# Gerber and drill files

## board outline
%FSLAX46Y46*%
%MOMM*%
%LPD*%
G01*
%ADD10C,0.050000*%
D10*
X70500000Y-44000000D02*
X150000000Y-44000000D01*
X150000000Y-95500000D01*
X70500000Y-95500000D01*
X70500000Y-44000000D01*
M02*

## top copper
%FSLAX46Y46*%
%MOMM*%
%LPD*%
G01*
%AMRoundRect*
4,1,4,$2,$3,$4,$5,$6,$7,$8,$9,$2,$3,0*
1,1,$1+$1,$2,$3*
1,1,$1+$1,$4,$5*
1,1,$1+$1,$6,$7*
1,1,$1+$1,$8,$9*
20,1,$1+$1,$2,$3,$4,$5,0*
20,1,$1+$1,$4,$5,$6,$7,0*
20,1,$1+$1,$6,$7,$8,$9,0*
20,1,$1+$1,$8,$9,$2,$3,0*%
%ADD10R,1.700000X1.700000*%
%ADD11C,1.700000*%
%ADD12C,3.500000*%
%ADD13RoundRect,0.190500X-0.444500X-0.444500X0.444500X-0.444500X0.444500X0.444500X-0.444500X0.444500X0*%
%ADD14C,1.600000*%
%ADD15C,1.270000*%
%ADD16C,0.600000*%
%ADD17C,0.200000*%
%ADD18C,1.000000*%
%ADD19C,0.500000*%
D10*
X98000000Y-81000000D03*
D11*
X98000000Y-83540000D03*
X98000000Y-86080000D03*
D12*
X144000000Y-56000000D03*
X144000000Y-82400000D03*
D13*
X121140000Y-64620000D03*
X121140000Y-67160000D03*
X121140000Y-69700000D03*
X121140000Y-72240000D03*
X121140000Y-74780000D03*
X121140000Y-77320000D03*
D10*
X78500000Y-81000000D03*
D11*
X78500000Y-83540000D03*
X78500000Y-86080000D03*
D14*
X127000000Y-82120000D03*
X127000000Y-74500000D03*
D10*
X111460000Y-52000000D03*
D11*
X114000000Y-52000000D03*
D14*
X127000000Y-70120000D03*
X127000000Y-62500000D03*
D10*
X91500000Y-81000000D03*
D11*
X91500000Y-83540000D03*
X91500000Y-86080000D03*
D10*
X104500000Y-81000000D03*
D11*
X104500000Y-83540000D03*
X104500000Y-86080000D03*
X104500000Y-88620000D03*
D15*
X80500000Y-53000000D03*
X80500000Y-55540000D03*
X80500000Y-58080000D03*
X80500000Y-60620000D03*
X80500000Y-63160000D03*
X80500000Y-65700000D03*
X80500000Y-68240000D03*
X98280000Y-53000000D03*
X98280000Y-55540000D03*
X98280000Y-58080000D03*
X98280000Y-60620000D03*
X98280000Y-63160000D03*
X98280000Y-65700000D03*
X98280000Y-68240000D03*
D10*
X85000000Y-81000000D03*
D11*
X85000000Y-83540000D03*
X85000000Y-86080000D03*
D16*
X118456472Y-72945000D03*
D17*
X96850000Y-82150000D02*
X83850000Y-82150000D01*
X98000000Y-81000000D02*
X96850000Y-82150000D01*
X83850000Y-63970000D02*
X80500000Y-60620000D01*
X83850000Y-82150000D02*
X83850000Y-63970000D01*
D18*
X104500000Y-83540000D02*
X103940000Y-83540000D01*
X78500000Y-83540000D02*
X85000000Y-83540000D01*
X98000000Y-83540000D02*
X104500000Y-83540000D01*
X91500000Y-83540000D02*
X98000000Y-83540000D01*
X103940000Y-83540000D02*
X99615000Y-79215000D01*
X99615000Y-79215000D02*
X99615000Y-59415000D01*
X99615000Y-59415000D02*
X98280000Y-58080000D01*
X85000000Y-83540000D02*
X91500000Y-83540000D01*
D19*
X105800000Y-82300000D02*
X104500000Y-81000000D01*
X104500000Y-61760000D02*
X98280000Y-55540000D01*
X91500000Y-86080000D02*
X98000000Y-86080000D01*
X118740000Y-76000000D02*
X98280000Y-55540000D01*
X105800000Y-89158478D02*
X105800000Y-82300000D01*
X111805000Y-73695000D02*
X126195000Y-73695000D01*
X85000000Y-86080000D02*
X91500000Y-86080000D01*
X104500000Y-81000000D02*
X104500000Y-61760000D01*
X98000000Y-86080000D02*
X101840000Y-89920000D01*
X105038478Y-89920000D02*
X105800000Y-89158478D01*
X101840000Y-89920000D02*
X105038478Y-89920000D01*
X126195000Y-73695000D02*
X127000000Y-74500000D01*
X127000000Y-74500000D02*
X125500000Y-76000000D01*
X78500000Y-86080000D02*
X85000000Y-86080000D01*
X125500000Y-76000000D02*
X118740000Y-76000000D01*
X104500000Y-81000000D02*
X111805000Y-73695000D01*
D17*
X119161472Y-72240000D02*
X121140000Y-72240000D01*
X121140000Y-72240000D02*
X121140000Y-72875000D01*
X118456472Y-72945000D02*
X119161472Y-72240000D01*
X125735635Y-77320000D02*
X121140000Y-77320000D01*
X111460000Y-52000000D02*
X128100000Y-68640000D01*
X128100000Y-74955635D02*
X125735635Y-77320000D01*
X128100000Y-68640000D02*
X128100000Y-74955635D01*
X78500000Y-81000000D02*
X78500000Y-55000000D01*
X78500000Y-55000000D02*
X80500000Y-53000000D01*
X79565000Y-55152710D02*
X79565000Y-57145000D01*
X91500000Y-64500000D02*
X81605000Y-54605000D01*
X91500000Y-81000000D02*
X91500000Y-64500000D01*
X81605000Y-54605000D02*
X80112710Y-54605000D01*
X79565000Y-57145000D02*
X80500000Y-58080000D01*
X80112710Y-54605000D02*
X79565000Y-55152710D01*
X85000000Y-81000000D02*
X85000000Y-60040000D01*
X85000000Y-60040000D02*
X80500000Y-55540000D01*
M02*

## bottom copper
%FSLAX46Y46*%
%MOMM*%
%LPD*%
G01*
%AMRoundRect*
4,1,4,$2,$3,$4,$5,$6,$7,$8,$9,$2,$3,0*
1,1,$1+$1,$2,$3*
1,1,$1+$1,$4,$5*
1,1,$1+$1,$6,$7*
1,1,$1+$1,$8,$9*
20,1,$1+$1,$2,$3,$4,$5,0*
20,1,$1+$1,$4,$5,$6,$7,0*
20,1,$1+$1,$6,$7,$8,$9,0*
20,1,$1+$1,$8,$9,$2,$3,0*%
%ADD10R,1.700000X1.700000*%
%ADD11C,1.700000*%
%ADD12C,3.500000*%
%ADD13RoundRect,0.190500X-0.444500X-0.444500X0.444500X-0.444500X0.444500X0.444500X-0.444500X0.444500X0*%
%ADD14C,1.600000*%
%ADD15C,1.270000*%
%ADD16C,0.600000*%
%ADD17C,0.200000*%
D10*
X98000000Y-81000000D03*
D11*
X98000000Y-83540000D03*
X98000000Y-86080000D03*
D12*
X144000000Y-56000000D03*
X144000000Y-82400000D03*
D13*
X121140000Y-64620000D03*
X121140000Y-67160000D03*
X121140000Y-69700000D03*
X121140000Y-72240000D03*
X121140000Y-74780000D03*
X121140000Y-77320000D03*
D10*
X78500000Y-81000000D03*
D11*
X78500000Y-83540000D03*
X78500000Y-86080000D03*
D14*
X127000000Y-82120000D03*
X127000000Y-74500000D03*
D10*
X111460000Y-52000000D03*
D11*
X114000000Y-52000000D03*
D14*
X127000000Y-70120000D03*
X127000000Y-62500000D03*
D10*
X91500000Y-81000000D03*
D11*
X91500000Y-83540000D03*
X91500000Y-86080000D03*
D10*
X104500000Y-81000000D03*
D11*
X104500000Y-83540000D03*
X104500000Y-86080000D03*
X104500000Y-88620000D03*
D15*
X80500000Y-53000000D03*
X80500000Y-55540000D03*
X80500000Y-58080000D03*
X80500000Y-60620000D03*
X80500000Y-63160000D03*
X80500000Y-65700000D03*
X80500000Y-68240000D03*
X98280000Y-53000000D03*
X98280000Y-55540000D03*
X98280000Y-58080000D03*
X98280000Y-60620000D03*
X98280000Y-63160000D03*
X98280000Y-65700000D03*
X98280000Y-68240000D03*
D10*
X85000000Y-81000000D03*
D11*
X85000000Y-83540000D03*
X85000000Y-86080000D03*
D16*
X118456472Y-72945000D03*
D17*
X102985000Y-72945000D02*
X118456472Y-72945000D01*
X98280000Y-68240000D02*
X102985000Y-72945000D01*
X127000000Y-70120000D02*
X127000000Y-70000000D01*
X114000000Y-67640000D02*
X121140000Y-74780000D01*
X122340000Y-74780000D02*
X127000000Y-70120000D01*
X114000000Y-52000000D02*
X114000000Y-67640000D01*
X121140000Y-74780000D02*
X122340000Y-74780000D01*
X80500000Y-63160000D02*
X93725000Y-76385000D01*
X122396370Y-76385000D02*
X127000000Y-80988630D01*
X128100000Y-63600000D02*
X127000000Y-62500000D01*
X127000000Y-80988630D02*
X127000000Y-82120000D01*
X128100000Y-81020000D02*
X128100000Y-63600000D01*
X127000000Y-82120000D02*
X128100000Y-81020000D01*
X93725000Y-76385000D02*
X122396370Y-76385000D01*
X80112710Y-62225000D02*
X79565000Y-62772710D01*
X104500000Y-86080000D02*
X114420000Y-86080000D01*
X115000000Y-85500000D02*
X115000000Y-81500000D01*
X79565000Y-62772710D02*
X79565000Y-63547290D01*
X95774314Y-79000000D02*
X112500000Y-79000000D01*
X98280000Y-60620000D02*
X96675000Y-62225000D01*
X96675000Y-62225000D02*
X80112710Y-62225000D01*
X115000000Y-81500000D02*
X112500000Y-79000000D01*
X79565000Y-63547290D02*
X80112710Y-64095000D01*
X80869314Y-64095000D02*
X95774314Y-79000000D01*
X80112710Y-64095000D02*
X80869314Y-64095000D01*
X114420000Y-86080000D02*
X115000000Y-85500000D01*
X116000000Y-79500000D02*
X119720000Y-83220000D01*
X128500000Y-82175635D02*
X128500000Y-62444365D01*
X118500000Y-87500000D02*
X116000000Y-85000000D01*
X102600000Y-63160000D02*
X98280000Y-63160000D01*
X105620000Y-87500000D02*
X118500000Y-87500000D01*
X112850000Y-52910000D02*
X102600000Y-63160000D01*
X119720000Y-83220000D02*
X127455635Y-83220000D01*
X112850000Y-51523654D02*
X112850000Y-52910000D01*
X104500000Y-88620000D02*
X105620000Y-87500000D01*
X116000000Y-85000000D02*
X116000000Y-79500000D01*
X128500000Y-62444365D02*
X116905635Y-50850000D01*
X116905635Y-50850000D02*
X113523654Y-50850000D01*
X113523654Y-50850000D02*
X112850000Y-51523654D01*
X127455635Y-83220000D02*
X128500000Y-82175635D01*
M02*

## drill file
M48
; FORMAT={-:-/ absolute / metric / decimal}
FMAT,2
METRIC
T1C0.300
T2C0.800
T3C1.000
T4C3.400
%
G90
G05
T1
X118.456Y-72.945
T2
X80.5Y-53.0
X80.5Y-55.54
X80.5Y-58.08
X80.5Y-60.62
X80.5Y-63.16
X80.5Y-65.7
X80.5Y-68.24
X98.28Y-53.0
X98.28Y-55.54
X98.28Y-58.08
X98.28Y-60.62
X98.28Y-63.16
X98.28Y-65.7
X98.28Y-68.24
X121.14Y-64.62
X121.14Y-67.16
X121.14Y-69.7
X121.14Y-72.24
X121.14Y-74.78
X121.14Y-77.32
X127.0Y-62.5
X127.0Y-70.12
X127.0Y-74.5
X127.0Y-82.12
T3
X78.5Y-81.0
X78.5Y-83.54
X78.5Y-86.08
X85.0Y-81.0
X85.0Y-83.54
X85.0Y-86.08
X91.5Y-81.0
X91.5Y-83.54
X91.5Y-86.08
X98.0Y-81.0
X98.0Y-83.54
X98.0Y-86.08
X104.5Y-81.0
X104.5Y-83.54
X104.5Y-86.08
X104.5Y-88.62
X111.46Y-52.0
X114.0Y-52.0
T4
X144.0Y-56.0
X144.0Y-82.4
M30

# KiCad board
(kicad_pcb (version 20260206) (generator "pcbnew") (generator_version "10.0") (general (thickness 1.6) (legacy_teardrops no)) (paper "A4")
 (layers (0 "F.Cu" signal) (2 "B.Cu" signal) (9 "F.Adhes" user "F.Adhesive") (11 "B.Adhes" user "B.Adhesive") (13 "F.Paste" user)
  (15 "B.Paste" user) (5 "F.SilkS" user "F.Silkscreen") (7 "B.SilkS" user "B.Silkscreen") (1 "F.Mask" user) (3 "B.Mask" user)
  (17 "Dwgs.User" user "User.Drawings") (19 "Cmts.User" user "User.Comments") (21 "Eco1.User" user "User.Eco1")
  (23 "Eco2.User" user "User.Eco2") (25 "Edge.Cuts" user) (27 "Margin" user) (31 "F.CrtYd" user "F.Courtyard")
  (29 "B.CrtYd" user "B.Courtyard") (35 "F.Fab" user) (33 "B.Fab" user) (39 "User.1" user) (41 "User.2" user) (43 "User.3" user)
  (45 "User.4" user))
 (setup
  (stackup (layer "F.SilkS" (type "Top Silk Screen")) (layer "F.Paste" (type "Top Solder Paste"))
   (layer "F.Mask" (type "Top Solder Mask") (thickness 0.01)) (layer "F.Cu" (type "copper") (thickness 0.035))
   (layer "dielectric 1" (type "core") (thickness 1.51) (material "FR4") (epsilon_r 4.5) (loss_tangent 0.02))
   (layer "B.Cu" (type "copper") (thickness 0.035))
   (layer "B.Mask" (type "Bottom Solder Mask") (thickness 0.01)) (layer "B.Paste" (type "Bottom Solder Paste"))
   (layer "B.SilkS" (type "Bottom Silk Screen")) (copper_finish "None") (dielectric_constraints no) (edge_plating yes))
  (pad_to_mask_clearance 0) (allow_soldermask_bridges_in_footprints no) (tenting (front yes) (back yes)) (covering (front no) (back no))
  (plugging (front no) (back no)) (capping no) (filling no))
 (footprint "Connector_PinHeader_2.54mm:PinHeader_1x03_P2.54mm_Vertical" (layer "F.Cu") (at 98 81)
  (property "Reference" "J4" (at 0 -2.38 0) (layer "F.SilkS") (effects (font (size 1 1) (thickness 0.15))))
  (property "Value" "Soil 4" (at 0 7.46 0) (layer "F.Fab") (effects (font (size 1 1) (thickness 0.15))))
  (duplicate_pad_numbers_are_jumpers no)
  (pad "1" thru_hole rect (at 0 0) (size 1.7 1.7) (drill 1) (layers "*.Cu" "*.Mask") (remove_unused_layers no) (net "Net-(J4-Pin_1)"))
  (pad "2" thru_hole circle (at 0 2.54) (size 1.7 1.7) (drill 1) (layers "*.Cu" "*.Mask") (remove_unused_layers no) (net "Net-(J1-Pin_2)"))
  (pad "3" thru_hole circle (at 0 5.08) (size 1.7 1.7) (drill 1) (layers "*.Cu" "*.Mask") (remove_unused_layers no) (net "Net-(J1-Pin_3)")))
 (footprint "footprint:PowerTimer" (layer "F.Cu") (at 126.22 59.54)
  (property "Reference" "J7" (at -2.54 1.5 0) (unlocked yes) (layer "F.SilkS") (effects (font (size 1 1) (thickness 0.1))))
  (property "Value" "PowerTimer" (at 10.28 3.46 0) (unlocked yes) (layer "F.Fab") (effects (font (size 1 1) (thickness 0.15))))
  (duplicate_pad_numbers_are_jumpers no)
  (pad "" np_thru_hole circle (at 17.78 -3.54) (size 3.5 3.5) (drill 3.4) (layers "*.Cu" "*.Mask"))
  (pad "" np_thru_hole circle (at 17.78 22.86) (size 3.5 3.5) (drill 3.4) (layers "*.Cu" "*.Mask"))
  (pad "1" thru_hole roundrect (at -5.08 5.08) (size 1.27 1.27) (drill 0.8) (layers "*.Cu" "*.Mask") (remove_unused_layers no)
   (roundrect_rratio 0.15) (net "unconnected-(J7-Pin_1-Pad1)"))
  (pad "2" thru_hole roundrect (at -5.08 7.62) (size 1.27 1.27) (drill 0.8) (layers "*.Cu" "*.Mask") (remove_unused_layers no)
   (roundrect_rratio 0.15) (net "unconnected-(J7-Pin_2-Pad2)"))
  (pad "3" thru_hole roundrect (at -5.08 10.16) (size 1.27 1.27) (drill 0.8) (layers "*.Cu" "*.Mask") (remove_unused_layers no)
   (roundrect_rratio 0.15) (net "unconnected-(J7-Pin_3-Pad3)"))
  (pad "4" thru_hole roundrect (at -5.08 12.7) (size 1.27 1.27) (drill 0.8) (layers "*.Cu" "*.Mask") (remove_unused_layers no)
   (roundrect_rratio 0.15) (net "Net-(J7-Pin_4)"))
  (pad "5" thru_hole roundrect (at -5.08 15.24) (size 1.27 1.27) (drill 0.8) (layers "*.Cu" "*.Mask") (remove_unused_layers no)
   (roundrect_rratio 0.15) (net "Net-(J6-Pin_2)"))
  (pad "6" thru_hole roundrect (at -5.08 17.78) (size 1.27 1.27) (drill 0.8) (layers "*.Cu" "*.Mask") (remove_unused_layers no)
   (roundrect_rratio 0.15) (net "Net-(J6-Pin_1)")))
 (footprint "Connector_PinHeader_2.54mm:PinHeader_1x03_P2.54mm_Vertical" (layer "F.Cu") (at 78.5 81)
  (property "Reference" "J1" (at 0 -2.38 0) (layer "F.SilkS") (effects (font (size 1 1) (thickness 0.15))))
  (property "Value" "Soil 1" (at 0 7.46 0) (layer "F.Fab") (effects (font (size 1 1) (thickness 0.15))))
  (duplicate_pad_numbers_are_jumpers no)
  (pad "1" thru_hole rect (at 0 0) (size 1.7 1.7) (drill 1) (layers "*.Cu" "*.Mask") (remove_unused_layers no) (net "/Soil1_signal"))
  (pad "2" thru_hole circle (at 0 2.54) (size 1.7 1.7) (drill 1) (layers "*.Cu" "*.Mask") (remove_unused_layers no) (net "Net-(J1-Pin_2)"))
  (pad "3" thru_hole circle (at 0 5.08) (size 1.7 1.7) (drill 1) (layers "*.Cu" "*.Mask") (remove_unused_layers no) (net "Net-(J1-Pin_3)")))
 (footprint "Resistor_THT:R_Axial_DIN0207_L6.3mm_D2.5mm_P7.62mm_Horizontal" (layer "F.Cu") (at 127 82.12 90)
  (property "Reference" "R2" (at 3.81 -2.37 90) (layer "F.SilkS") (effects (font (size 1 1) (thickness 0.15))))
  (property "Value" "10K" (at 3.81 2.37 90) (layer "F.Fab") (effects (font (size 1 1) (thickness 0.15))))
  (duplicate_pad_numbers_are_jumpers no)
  (pad "1" thru_hole circle (at 0 0 90) (size 1.6 1.6) (drill 0.8) (layers "*.Cu" "*.Mask") (remove_unused_layers no) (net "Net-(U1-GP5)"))
  (pad "2" thru_hole circle (at 7.62 0 90) (size 1.6 1.6) (drill 0.8) (layers "*.Cu" "*.Mask") (remove_unused_layers no)
   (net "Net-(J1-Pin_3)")))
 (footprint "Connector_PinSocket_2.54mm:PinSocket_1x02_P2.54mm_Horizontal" (layer "F.Cu") (at 111.46 52 90)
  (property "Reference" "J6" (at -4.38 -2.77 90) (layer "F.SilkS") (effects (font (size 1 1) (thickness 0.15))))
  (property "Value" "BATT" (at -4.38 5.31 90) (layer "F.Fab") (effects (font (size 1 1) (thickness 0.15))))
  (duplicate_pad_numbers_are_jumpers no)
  (pad "1" thru_hole rect (at 0 0 90) (size 1.7 1.7) (drill 1) (layers "*.Cu" "*.Mask") (remove_unused_layers no) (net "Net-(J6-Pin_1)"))
  (pad "2" thru_hole circle (at 0 2.54 90) (size 1.7 1.7) (drill 1) (layers "*.Cu" "*.Mask") (remove_unused_layers no)
   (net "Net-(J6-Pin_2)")))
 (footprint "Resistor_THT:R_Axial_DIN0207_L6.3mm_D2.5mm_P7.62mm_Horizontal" (layer "F.Cu") (at 127 70.12 90)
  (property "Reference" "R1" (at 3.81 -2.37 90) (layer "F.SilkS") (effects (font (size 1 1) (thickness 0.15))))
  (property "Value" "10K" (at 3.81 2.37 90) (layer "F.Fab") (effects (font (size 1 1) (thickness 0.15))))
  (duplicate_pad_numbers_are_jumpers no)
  (pad "1" thru_hole circle (at 0 0 90) (size 1.6 1.6) (drill 0.8) (layers "*.Cu" "*.Mask") (remove_unused_layers no) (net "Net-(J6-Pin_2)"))
  (pad "2" thru_hole circle (at 7.62 0 90) (size 1.6 1.6) (drill 0.8) (layers "*.Cu" "*.Mask") (remove_unused_layers no)
   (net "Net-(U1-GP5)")))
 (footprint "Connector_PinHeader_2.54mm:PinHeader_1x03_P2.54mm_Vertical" (layer "F.Cu") (at 91.5 81)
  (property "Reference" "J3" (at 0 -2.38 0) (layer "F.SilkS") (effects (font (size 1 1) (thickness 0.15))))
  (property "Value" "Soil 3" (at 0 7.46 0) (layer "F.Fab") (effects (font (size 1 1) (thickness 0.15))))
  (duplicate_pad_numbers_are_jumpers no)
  (pad "1" thru_hole rect (at 0 0) (size 1.7 1.7) (drill 1) (layers "*.Cu" "*.Mask") (remove_unused_layers no) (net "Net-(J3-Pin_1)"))
  (pad "2" thru_hole circle (at 0 2.54) (size 1.7 1.7) (drill 1) (layers "*.Cu" "*.Mask") (remove_unused_layers no) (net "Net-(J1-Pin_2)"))
  (pad "3" thru_hole circle (at 0 5.08) (size 1.7 1.7) (drill 1) (layers "*.Cu" "*.Mask") (remove_unused_layers no) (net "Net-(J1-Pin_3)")))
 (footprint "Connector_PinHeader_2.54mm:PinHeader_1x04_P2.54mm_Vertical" (layer "F.Cu") (at 104.5 81)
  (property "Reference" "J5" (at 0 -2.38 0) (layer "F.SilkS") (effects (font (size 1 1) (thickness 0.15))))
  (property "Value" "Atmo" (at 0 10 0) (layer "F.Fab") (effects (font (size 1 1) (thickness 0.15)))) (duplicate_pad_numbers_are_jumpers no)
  (pad "1" thru_hole rect (at 0 0) (size 1.7 1.7) (drill 1) (layers "*.Cu" "*.Mask") (remove_unused_layers no) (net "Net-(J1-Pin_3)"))
  (pad "2" thru_hole circle (at 0 2.54) (size 1.7 1.7) (drill 1) (layers "*.Cu" "*.Mask") (remove_unused_layers no) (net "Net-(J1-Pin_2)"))
  (pad "3" thru_hole circle (at 0 5.08) (size 1.7 1.7) (drill 1) (layers "*.Cu" "*.Mask") (remove_unused_layers no) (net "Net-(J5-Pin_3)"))
  (pad "4" thru_hole circle (at 0 7.62) (size 1.7 1.7) (drill 1) (layers "*.Cu" "*.Mask") (remove_unused_layers no) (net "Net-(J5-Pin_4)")))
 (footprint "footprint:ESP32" (layer "F.Cu") (at 80.5 53)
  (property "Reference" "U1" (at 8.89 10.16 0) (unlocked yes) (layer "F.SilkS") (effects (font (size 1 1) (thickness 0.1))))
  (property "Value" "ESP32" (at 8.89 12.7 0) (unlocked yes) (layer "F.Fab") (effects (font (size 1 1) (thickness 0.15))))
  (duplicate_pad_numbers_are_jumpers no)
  (pad "1" thru_hole circle (at 0 0) (size 1.27 1.27) (drill 0.8) (layers "*.Cu" "*.Mask") (remove_unused_layers no) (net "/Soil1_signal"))
  (pad "2" thru_hole circle (at 0 2.54) (size 1.27 1.27) (drill 0.8) (layers "*.Cu" "*.Mask") (remove_unused_layers no)
   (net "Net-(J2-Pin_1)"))
  (pad "3" thru_hole circle (at 0 5.08) (size 1.27 1.27) (drill 0.8) (layers "*.Cu" "*.Mask") (remove_unused_layers no)
   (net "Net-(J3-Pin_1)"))
  (pad "4" thru_hole circle (at 0 7.62) (size 1.27 1.27) (drill 0.8) (layers "*.Cu" "*.Mask") (remove_unused_layers no)
   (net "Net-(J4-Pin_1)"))
  (pad "5" thru_hole circle (at 0 10.16) (size 1.27 1.27) (drill 0.8) (layers "*.Cu" "*.Mask") (remove_unused_layers no)
   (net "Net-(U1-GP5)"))
  (pad "6" thru_hole circle (at 0 12.7) (size 1.27 1.27) (drill 0.8) (layers "*.Cu" "*.Mask") (remove_unused_layers no)
   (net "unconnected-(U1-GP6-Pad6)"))
  (pad "7" thru_hole circle (at 0 15.24) (size 1.27 1.27) (drill 0.8) (layers "*.Cu" "*.Mask") (remove_unused_layers no)
   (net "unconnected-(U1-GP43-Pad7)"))
  (pad "8" thru_hole circle (at 17.78 0) (size 1.27 1.27) (drill 0.8) (layers "*.Cu" "*.Mask") (remove_unused_layers no)
   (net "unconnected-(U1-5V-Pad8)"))
  (pad "9" thru_hole circle (at 17.78 2.54) (size 1.27 1.27) (drill 0.8) (layers "*.Cu" "*.Mask") (remove_unused_layers no)
   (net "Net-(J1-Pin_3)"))
  (pad "10" thru_hole circle (at 17.78 5.08) (size 1.27 1.27) (drill 0.8) (layers "*.Cu" "*.Mask") (remove_unused_layers no)
   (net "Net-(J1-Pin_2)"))
  (pad "11" thru_hole circle (at 17.78 7.62) (size 1.27 1.27) (drill 0.8) (layers "*.Cu" "*.Mask") (remove_unused_layers no)
   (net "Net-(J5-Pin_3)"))
  (pad "12" thru_hole circle (at 17.78 10.16) (size 1.27 1.27) (drill 0.8) (layers "*.Cu" "*.Mask") (remove_unused_layers no)
   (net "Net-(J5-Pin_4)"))
  (pad "13" thru_hole circle (at 17.78 12.7) (size 1.27 1.27) (drill 0.8) (layers "*.Cu" "*.Mask") (remove_unused_layers no)
   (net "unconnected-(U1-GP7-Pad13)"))
  (pad "14" thru_hole circle (at 17.78 15.24) (size 1.27 1.27) (drill 0.8) (layers "*.Cu" "*.Mask") (remove_unused_layers no)
   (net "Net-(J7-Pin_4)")))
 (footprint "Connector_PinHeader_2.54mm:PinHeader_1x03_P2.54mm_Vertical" (layer "F.Cu") (at 85 81)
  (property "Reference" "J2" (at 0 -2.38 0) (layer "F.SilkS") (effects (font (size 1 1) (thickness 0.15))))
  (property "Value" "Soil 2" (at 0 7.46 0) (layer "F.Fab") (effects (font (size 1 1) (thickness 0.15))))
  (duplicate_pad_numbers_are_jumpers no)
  (pad "1" thru_hole rect (at 0 0) (size 1.7 1.7) (drill 1) (layers "*.Cu" "*.Mask") (remove_unused_layers no) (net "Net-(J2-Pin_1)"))
  (pad "2" thru_hole circle (at 0 2.54) (size 1.7 1.7) (drill 1) (layers "*.Cu" "*.Mask") (remove_unused_layers no) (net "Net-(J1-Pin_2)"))
  (pad "3" thru_hole circle (at 0 5.08) (size 1.7 1.7) (drill 1) (layers "*.Cu" "*.Mask") (remove_unused_layers no) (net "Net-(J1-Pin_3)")))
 (gr_rect (start 70.5 44) (end 150 95.5) (stroke (width 0.05) (type default)) (fill no) (layer "Edge.Cuts"))
 (segment (start 96.85 82.15) (end 83.85 82.15) (width 0.2) (layer "F.Cu") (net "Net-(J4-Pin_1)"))
 (segment (start 98 81) (end 96.85 82.15) (width 0.2) (layer "F.Cu") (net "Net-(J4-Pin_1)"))
 (segment (start 83.85 63.97) (end 80.5 60.62) (width 0.2) (layer "F.Cu") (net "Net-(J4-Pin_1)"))
 (segment (start 83.85 82.15) (end 83.85 63.97) (width 0.2) (layer "F.Cu") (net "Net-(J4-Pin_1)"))
 (segment (start 104.5 83.54) (end 103.94 83.54) (width 1) (layer "F.Cu") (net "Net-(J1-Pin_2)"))
 (segment (start 78.5 83.54) (end 85 83.54) (width 1) (layer "F.Cu") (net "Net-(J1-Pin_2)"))
 (segment (start 98 83.54) (end 104.5 83.54) (width 1) (layer "F.Cu") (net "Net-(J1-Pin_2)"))
 (segment (start 91.5 83.54) (end 98 83.54) (width 1) (layer "F.Cu") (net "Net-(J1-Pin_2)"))
 (segment (start 103.94 83.54) (end 99.615 79.215) (width 1) (layer "F.Cu") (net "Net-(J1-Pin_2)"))
 (segment (start 99.615 79.215) (end 99.615 59.415) (width 1) (layer "F.Cu") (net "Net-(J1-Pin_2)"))
 (segment (start 99.615 59.415) (end 98.28 58.08) (width 1) (layer "F.Cu") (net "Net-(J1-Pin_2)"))
 (segment (start 85 83.54) (end 91.5 83.54) (width 1) (layer "F.Cu") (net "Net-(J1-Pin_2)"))
 (segment (start 105.8 82.3) (end 104.5 81) (width 0.5) (layer "F.Cu") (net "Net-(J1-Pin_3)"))
 (segment (start 104.5 61.76) (end 98.28 55.54) (width 0.5) (layer "F.Cu") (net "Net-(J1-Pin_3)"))
 (segment (start 91.5 86.08) (end 98 86.08) (width 0.5) (layer "F.Cu") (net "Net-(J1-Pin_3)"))
 (segment (start 118.74 76) (end 98.28 55.54) (width 0.5) (layer "F.Cu") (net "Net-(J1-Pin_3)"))
 (segment (start 105.8 89.158478) (end 105.8 82.3) (width 0.5) (layer "F.Cu") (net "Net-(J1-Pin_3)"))
 (segment (start 111.805 73.695) (end 126.195 73.695) (width 0.5) (layer "F.Cu") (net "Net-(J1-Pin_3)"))
 (segment (start 85 86.08) (end 91.5 86.08) (width 0.5) (layer "F.Cu") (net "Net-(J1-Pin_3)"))
 (segment (start 104.5 81) (end 104.5 61.76) (width 0.5) (layer "F.Cu") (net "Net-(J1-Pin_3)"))
 (segment (start 98 86.08) (end 101.84 89.92) (width 0.5) (layer "F.Cu") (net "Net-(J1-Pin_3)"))
 (segment (start 105.038478 89.92) (end 105.8 89.158478) (width 0.5) (layer "F.Cu") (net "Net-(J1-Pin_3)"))
 (segment (start 101.84 89.92) (end 105.038478 89.92) (width 0.5) (layer "F.Cu") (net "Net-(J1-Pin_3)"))
 (segment (start 126.195 73.695) (end 127 74.5) (width 0.5) (layer "F.Cu") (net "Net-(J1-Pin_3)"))
 (segment (start 127 74.5) (end 125.5 76) (width 0.5) (layer "F.Cu") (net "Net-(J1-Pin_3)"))
 (segment (start 78.5 86.08) (end 85 86.08) (width 0.5) (layer "F.Cu") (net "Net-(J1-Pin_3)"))
 (segment (start 125.5 76) (end 118.74 76) (width 0.5) (layer "F.Cu") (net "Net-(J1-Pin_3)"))
 (segment (start 104.5 81) (end 111.805 73.695) (width 0.5) (layer "F.Cu") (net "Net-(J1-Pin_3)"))
 (segment (start 119.161472 72.24) (end 121.14 72.24) (width 0.2) (layer "F.Cu") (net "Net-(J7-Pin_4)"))
 (segment (start 121.14 72.24) (end 121.14 72.875) (width 0.2) (layer "F.Cu") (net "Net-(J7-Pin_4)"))
 (segment (start 118.456472 72.945) (end 119.161472 72.24) (width 0.2) (layer "F.Cu") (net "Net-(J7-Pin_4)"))
 (via (at 118.456472 72.945) (size 0.6) (drill 0.3) (layers "F.Cu" "B.Cu") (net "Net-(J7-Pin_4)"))
 (segment (start 102.985 72.945) (end 118.456472 72.945) (width 0.2) (layer "B.Cu") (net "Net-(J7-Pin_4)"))
 (segment (start 98.28 68.24) (end 102.985 72.945) (width 0.2) (layer "B.Cu") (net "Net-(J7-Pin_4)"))
 (segment (start 127 70.12) (end 127 70) (width 0.2) (layer "B.Cu") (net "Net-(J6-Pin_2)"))
 (segment (start 114 67.64) (end 121.14 74.78) (width 0.2) (layer "B.Cu") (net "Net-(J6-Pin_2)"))
 (segment (start 122.34 74.78) (end 127 70.12) (width 0.2) (layer "B.Cu") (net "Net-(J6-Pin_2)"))
 (segment (start 114 52) (end 114 67.64) (width 0.2) (layer "B.Cu") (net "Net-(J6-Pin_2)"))
 (segment (start 121.14 74.78) (end 122.34 74.78) (width 0.2) (layer "B.Cu") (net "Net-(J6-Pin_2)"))
 (segment (start 125.735635 77.32) (end 121.14 77.32) (width 0.2) (layer "F.Cu") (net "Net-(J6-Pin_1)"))
 (segment (start 111.46 52) (end 128.1 68.64) (width 0.2) (layer "F.Cu") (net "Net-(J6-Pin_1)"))
 (segment (start 128.1 74.955635) (end 125.735635 77.32) (width 0.2) (layer "F.Cu") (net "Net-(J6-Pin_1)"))
 (segment (start 128.1 68.64) (end 128.1 74.955635) (width 0.2) (layer "F.Cu") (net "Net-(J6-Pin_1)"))
 (segment (start 78.5 81) (end 78.5 55) (width 0.2) (layer "F.Cu") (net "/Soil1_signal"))
 (segment (start 78.5 55) (end 80.5 53) (width 0.2) (layer "F.Cu") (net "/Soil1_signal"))
 (segment (start 80.5 63.16) (end 93.725 76.385) (width 0.2) (layer "B.Cu") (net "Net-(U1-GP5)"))
 (segment (start 122.39637 76.385) (end 127 80.98863) (width 0.2) (layer "B.Cu") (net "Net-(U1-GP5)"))
 (segment (start 128.1 63.6) (end 127 62.5) (width 0.2) (layer "B.Cu") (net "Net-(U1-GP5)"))
 (segment (start 127 80.98863) (end 127 82.12) (width 0.2) (layer "B.Cu") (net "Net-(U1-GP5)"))
 (segment (start 128.1 81.02) (end 128.1 63.6) (width 0.2) (layer "B.Cu") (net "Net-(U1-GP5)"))
 (segment (start 127 82.12) (end 128.1 81.02) (width 0.2) (layer "B.Cu") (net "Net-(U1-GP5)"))
 (segment (start 93.725 76.385) (end 122.39637 76.385) (width 0.2) (layer "B.Cu") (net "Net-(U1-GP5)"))
 (segment (start 79.565 55.15271) (end 79.565 57.145) (width 0.2) (layer "F.Cu") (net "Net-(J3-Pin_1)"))
 (segment (start 91.5 64.5) (end 81.605 54.605) (width 0.2) (layer "F.Cu") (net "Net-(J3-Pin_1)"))
 (segment (start 91.5 81) (end 91.5 64.5) (width 0.2) (layer "F.Cu") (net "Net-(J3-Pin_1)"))
 (segment (start 81.605 54.605) (end 80.11271 54.605) (width 0.2) (layer "F.Cu") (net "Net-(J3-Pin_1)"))
 (segment (start 79.565 57.145) (end 80.5 58.08) (width 0.2) (layer "F.Cu") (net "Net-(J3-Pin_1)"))
 (segment (start 80.11271 54.605) (end 79.565 55.15271) (width 0.2) (layer "F.Cu") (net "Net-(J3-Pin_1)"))
 (segment (start 80.11271 62.225) (end 79.565 62.77271) (width 0.2) (layer "B.Cu") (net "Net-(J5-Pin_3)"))
 (segment (start 104.5 86.08) (end 114.42 86.08) (width 0.2) (layer "B.Cu") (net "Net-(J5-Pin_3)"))
 (segment (start 115 85.5) (end 115 81.5) (width 0.2) (layer "B.Cu") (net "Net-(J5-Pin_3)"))
 (segment (start 79.565 62.77271) (end 79.565 63.54729) (width 0.2) (layer "B.Cu") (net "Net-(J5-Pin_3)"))
 (segment (start 95.774314 79) (end 112.5 79) (width 0.2) (layer "B.Cu") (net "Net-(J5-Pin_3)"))
 (segment (start 98.28 60.62) (end 96.675 62.225) (width 0.2) (layer "B.Cu") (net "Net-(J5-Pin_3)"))
 (segment (start 96.675 62.225) (end 80.11271 62.225) (width 0.2) (layer "B.Cu") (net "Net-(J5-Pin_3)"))
 (segment (start 115 81.5) (end 112.5 79) (width 0.2) (layer "B.Cu") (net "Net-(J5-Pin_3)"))
 (segment (start 79.565 63.54729) (end 80.11271 64.095) (width 0.2) (layer "B.Cu") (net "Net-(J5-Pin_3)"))
 (segment (start 80.869314 64.095) (end 95.774314 79) (width 0.2) (layer "B.Cu") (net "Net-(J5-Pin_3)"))
 (segment (start 80.11271 64.095) (end 80.869314 64.095) (width 0.2) (layer "B.Cu") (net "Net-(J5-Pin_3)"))
 (segment (start 114.42 86.08) (end 115 85.5) (width 0.2) (layer "B.Cu") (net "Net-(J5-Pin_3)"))
 (segment (start 116 79.5) (end 119.72 83.22) (width 0.2) (layer "B.Cu") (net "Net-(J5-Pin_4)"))
 (segment (start 128.5 82.175635) (end 128.5 62.444365) (width 0.2) (layer "B.Cu") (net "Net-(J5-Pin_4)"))
 (segment (start 118.5 87.5) (end 116 85) (width 0.2) (layer "B.Cu") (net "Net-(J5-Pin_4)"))
 (segment (start 102.6 63.16) (end 98.28 63.16) (width 0.2) (layer "B.Cu") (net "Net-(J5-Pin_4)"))
 (segment (start 105.62 87.5) (end 118.5 87.5) (width 0.2) (layer "B.Cu") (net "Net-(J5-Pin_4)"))
 (segment (start 112.85 52.91) (end 102.6 63.16) (width 0.2) (layer "B.Cu") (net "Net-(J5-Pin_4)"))
 (segment (start 119.72 83.22) (end 127.455635 83.22) (width 0.2) (layer "B.Cu") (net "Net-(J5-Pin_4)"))
 (segment (start 112.85 51.523654) (end 112.85 52.91) (width 0.2) (layer "B.Cu") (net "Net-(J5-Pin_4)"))
 (segment (start 104.5 88.62) (end 105.62 87.5) (width 0.2) (layer "B.Cu") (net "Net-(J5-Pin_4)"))
 (segment (start 116 85) (end 116 79.5) (width 0.2) (layer "B.Cu") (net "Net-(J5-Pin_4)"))
 (segment (start 128.5 62.444365) (end 116.905635 50.85) (width 0.2) (layer "B.Cu") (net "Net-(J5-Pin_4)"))
 (segment (start 116.905635 50.85) (end 113.523654 50.85) (width 0.2) (layer "B.Cu") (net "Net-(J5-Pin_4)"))
 (segment (start 113.523654 50.85) (end 112.85 51.523654) (width 0.2) (layer "B.Cu") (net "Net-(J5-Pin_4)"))
 (segment (start 127.455635 83.22) (end 128.5 82.175635) (width 0.2) (layer "B.Cu") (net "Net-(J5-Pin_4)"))
 (segment (start 85 81) (end 85 60.04) (width 0.2) (layer "F.Cu") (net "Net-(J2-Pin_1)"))
 (segment (start 85 60.04) (end 80.5 55.54) (width 0.2) (layer "F.Cu") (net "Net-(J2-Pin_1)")))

